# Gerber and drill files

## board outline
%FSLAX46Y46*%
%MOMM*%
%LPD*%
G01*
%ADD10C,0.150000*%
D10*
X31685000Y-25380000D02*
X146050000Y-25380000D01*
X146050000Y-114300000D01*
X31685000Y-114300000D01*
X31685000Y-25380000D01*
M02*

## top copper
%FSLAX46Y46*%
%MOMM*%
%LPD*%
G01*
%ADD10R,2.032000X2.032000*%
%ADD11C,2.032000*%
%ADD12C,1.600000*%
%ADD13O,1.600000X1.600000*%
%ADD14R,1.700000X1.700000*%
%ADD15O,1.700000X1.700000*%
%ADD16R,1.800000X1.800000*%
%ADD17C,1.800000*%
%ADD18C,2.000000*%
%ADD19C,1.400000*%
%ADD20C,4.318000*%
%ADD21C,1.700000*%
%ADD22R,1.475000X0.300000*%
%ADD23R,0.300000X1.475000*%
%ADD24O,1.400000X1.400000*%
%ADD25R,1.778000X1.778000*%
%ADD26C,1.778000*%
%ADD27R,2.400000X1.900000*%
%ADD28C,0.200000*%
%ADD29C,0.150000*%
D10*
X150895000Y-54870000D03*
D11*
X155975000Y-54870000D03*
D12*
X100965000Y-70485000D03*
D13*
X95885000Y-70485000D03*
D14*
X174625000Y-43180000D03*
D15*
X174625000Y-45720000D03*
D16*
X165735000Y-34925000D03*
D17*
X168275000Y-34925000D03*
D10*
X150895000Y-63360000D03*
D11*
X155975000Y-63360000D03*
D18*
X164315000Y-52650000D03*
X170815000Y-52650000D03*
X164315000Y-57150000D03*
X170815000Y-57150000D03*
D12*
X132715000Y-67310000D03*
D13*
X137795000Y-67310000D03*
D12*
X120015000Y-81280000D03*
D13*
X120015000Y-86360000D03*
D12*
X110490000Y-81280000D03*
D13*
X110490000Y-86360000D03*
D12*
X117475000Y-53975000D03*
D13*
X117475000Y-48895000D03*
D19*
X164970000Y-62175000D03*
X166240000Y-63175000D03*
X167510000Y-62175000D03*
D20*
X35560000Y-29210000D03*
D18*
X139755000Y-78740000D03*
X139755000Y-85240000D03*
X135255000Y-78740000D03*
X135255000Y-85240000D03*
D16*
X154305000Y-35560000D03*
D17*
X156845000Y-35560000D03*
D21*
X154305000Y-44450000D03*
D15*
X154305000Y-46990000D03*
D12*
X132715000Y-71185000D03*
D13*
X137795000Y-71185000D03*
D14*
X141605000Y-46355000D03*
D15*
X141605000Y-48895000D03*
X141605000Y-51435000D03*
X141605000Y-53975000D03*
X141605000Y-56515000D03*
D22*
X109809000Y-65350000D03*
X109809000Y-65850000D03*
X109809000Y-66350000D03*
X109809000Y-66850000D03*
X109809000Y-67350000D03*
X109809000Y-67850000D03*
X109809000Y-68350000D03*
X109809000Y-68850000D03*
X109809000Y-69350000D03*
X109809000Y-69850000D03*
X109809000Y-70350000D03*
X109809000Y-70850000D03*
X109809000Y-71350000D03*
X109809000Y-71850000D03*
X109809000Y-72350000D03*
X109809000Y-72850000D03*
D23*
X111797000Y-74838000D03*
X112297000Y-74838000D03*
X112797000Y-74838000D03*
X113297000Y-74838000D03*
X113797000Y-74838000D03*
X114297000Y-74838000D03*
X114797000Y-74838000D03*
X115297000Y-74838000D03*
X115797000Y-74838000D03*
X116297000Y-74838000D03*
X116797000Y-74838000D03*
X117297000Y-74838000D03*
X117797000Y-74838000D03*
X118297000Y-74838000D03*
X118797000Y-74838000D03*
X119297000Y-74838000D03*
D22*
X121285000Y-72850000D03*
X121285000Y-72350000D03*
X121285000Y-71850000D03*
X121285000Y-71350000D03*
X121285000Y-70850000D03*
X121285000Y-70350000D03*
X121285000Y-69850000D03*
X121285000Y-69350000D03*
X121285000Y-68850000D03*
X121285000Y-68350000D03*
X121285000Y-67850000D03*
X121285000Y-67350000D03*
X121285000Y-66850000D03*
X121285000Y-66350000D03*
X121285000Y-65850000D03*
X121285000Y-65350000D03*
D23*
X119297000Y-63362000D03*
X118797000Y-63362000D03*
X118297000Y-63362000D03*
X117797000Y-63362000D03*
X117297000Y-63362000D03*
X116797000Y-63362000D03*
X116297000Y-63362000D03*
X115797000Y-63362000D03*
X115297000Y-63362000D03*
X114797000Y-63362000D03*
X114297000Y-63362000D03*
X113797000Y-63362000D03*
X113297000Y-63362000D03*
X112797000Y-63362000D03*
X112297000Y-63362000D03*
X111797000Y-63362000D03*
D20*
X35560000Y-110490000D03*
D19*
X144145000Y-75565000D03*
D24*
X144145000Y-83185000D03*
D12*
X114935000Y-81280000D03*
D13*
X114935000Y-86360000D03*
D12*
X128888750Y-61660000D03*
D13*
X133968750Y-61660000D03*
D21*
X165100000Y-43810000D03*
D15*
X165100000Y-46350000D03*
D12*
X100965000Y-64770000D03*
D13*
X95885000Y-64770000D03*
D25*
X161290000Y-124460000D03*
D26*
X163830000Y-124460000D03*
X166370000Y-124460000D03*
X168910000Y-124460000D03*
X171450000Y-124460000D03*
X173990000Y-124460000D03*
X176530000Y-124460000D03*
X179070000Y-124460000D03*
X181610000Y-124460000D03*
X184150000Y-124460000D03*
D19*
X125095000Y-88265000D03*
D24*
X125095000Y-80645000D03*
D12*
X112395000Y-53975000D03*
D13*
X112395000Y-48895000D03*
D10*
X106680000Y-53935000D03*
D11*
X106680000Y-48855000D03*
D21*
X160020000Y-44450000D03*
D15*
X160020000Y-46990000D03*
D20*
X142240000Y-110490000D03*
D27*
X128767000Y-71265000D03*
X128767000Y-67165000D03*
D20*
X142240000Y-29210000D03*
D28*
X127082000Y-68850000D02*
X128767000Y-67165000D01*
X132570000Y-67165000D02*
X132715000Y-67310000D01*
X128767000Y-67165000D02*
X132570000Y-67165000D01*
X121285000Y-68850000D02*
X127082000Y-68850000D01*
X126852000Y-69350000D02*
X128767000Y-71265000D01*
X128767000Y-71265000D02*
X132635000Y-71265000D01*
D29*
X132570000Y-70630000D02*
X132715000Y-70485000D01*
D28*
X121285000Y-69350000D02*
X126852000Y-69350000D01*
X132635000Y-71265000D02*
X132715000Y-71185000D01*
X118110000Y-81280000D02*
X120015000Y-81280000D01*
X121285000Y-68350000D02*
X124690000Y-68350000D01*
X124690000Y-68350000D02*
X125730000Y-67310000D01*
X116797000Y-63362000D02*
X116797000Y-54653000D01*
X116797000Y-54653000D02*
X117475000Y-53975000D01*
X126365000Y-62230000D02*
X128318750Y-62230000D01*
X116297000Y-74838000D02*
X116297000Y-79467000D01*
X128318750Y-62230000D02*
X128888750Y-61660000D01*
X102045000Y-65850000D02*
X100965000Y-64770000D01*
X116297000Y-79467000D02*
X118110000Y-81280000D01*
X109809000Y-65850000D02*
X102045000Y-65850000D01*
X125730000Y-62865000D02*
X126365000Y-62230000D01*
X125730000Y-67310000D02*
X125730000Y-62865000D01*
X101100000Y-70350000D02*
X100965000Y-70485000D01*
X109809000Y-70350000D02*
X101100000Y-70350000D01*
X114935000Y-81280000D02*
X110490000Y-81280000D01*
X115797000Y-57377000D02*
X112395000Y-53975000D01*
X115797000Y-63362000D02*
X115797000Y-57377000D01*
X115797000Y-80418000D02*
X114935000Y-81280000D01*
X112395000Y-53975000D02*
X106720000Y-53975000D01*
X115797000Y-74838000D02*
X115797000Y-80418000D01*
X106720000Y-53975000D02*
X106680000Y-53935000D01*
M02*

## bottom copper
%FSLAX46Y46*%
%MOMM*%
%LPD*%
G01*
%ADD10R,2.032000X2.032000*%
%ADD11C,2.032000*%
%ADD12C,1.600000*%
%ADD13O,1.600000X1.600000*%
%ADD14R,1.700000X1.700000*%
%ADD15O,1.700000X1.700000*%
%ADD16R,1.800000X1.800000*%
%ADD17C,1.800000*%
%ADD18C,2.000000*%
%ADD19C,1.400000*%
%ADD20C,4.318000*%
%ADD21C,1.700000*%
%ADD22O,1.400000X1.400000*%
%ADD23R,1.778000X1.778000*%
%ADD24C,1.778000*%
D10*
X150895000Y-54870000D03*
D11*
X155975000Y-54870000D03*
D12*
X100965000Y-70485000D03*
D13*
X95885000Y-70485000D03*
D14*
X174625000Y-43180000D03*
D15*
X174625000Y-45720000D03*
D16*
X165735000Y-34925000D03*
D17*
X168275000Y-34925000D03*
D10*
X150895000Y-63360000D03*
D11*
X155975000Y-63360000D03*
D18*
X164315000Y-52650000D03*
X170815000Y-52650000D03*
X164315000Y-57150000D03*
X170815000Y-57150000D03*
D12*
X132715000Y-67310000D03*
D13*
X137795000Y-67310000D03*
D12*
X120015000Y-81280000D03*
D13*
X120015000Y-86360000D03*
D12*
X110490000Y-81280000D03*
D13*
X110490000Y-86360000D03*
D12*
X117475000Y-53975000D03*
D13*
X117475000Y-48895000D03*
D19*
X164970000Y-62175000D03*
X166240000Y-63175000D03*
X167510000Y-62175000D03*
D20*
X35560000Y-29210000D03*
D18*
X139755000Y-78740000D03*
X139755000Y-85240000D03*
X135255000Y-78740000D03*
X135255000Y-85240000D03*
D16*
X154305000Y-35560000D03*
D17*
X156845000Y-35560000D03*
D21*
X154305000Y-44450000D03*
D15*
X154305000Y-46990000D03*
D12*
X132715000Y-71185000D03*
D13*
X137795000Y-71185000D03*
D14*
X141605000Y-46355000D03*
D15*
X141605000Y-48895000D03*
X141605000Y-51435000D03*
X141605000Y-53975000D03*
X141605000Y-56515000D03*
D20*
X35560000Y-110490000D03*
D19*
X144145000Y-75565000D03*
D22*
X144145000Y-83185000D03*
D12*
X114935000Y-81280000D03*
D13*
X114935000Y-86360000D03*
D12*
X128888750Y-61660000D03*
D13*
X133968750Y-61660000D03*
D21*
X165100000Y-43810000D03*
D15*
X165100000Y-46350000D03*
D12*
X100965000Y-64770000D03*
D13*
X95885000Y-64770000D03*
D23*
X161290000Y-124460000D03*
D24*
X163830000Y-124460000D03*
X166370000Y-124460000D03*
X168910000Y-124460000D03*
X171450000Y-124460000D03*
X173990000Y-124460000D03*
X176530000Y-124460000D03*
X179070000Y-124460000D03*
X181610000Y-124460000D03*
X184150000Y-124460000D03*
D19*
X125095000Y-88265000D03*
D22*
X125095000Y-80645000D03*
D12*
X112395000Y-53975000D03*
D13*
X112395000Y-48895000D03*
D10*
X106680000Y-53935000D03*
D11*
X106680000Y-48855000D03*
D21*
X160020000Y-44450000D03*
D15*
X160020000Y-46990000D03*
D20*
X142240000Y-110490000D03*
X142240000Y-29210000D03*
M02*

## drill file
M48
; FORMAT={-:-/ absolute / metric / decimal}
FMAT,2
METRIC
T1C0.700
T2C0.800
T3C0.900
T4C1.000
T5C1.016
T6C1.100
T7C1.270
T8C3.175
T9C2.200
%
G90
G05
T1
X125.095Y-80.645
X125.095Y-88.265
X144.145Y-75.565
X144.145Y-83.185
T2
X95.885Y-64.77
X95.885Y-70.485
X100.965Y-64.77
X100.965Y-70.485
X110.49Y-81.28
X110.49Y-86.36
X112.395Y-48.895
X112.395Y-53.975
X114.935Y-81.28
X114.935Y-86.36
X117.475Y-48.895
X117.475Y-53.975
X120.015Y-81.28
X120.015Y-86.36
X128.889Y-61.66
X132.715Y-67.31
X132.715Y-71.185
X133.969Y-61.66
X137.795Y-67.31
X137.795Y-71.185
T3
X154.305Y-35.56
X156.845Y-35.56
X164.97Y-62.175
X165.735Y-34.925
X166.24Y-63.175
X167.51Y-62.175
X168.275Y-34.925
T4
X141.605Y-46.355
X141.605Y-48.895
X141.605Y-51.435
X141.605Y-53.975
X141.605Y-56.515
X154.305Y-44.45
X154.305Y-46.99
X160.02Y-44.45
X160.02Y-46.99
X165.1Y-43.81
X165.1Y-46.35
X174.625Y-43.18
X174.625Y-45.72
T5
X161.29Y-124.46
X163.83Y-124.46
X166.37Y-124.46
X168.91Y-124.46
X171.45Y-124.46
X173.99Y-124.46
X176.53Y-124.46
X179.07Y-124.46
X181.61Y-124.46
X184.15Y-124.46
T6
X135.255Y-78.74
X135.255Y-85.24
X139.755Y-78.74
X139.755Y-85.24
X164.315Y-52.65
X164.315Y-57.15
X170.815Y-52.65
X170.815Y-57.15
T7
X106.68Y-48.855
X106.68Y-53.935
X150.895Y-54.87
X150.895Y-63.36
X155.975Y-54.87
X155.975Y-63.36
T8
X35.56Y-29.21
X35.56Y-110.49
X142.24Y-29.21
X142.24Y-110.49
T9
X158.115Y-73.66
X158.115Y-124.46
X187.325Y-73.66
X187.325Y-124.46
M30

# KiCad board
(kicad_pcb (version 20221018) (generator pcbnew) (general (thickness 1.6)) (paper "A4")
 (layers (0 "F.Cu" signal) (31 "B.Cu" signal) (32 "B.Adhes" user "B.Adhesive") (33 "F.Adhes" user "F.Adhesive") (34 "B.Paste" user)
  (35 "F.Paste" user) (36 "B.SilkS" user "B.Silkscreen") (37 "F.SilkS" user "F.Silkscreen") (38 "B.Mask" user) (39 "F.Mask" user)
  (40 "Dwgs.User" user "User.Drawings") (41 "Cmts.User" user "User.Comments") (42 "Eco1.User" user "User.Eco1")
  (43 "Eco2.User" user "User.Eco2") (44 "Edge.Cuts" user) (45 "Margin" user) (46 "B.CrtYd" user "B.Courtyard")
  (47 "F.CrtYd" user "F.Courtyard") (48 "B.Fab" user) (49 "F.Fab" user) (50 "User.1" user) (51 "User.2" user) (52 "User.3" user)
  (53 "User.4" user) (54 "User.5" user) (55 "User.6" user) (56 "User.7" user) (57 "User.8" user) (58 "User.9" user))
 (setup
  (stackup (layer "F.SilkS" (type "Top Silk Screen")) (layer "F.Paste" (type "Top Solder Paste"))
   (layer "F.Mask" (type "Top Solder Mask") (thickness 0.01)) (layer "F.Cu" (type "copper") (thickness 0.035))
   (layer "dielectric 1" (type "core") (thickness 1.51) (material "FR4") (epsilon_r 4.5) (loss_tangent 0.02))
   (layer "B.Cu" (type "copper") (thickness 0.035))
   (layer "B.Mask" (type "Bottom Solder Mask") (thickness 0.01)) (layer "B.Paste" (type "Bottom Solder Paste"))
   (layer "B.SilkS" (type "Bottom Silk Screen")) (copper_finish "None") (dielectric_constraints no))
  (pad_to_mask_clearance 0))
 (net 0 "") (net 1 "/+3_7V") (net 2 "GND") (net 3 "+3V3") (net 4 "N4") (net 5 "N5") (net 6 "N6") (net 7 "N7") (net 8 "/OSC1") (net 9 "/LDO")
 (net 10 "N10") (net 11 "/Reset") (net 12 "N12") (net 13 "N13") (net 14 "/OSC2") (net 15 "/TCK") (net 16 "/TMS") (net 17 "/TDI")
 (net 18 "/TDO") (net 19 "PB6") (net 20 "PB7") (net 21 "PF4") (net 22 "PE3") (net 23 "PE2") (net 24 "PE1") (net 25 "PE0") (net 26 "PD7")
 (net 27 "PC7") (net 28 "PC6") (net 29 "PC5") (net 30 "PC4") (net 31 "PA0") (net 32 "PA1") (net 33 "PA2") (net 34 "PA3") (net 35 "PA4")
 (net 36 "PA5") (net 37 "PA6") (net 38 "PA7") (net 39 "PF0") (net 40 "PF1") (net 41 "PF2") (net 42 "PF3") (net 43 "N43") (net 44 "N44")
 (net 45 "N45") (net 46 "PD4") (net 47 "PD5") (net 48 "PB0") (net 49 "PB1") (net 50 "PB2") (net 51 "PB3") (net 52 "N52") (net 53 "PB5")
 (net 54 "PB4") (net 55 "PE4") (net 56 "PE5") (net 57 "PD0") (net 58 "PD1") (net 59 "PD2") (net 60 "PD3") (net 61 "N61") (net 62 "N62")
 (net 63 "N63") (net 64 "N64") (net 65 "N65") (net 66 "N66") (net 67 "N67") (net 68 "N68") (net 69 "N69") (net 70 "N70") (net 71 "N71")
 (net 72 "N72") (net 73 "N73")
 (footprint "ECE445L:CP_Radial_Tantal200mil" (layer "F.Cu") (at 150.895 54.87)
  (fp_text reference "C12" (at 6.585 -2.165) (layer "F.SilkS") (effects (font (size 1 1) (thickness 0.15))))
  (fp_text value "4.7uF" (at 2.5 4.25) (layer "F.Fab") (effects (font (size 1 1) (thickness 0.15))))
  (pad "1" thru_hole rect (at 0 0) (size 2.032 2.032) (drill 1.27) (layers "*.Cu" "*.Mask") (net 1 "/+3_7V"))
  (pad "2" thru_hole circle (at 5.08 0) (size 2.032 2.032) (drill 1.27) (layers "*.Cu" "*.Mask") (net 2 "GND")))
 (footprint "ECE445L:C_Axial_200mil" (layer "F.Cu") (at 100.965 70.485 180)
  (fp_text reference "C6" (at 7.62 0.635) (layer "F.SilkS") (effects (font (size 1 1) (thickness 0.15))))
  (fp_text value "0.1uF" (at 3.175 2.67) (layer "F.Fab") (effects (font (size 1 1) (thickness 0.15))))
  (pad "1" thru_hole circle (at 0 0 180) (size 1.6 1.6) (drill 0.8) (layers "*.Cu" "*.Mask") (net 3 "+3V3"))
  (pad "2" thru_hole oval (at 5.08 0 180) (size 1.6 1.6) (drill 0.8) (layers "*.Cu" "*.Mask") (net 2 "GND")))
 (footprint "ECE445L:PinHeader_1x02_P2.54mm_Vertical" (layer "F.Cu") (at 174.625 43.18)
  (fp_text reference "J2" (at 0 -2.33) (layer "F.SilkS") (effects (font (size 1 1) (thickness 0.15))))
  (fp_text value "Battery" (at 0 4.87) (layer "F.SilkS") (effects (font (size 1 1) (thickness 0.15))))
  (pad "1" thru_hole rect (at 0 0) (size 1.7 1.7) (drill 1) (layers "*.Cu" "*.Mask") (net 2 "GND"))
  (pad "2" thru_hole oval (at 0 2.54) (size 1.7 1.7) (drill 1) (layers "*.Cu" "*.Mask") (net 1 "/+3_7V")))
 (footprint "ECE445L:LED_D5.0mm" (layer "F.Cu") (at 165.735 34.925)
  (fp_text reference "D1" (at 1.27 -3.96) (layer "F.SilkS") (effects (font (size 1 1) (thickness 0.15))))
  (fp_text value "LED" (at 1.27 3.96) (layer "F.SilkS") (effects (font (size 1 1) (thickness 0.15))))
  (pad "1" thru_hole rect (at 0 0) (size 1.8 1.8) (drill 0.9) (layers "*.Cu" "*.Mask") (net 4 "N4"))
  (pad "2" thru_hole circle (at 2.54 0) (size 1.8 1.8) (drill 0.9) (layers "*.Cu" "*.Mask") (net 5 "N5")))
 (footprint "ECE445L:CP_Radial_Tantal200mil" (layer "F.Cu") (at 150.895 63.36)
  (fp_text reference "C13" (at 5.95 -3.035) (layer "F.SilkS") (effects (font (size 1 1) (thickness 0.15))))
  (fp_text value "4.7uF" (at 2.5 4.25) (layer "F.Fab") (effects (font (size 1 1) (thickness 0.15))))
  (pad "1" thru_hole rect (at 0 0) (size 2.032 2.032) (drill 1.27) (layers "*.Cu" "*.Mask") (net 3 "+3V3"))
  (pad "2" thru_hole circle (at 5.08 0) (size 2.032 2.032) (drill 1.27) (layers "*.Cu" "*.Mask") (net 2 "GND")))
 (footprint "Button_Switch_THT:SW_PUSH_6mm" (layer "F.Cu") (at 164.315 52.65)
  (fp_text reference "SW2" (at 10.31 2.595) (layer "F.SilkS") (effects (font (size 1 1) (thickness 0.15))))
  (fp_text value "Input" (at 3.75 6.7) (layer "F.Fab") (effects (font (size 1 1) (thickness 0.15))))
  (pad "1" thru_hole circle (at 0 0 90) (size 2 2) (drill 1.1) (layers "*.Cu" "*.Mask") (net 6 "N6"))
  (pad "1" thru_hole circle (at 6.5 0 90) (size 2 2) (drill 1.1) (layers "*.Cu" "*.Mask") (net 6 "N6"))
  (pad "2" thru_hole circle (at 0 4.5 90) (size 2 2) (drill 1.1) (layers "*.Cu" "*.Mask") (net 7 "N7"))
  (pad "2" thru_hole circle (at 6.5 4.5 90) (size 2 2) (drill 1.1) (layers "*.Cu" "*.Mask") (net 7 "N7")))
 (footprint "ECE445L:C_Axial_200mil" (layer "F.Cu") (at 132.715 67.31)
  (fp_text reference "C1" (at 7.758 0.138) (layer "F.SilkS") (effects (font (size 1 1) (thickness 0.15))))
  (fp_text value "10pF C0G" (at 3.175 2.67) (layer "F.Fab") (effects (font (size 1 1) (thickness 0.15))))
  (pad "1" thru_hole circle (at 0 0) (size 1.6 1.6) (drill 0.8) (layers "*.Cu" "*.Mask") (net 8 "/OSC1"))
  (pad "2" thru_hole oval (at 5.08 0) (size 1.6 1.6) (drill 0.8) (layers "*.Cu" "*.Mask") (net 2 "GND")))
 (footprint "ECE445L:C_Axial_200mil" (layer "F.Cu") (at 120.015 81.28 -90)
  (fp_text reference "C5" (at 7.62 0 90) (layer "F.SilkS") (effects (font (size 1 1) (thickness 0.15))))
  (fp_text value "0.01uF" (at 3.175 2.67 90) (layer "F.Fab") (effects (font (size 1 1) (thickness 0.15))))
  (pad "1" thru_hole circle (at 0 0 270) (size 1.6 1.6) (drill 0.8) (layers "*.Cu" "*.Mask") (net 3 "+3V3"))
  (pad "2" thru_hole oval (at 5.08 0 270) (size 1.6 1.6) (drill 0.8) (layers "*.Cu" "*.Mask") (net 2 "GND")))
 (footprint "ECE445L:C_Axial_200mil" (layer "F.Cu") (at 110.49 81.28 -90)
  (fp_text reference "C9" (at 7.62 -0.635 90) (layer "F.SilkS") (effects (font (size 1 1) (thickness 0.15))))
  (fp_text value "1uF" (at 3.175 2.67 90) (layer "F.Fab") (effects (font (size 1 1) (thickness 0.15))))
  (pad "1" thru_hole circle (at 0 0 270) (size 1.6 1.6) (drill 0.8) (layers "*.Cu" "*.Mask") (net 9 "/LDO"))
  (pad "2" thru_hole oval (at 5.08 0 270) (size 1.6 1.6) (drill 0.8) (layers "*.Cu" "*.Mask") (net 2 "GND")))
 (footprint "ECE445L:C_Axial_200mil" (layer "F.Cu") (at 117.475 53.975 90)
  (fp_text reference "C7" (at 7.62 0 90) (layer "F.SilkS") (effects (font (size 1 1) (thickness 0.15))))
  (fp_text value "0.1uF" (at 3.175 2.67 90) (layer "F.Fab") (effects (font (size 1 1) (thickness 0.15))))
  (pad "1" thru_hole circle (at 0 0 90) (size 1.6 1.6) (drill 0.8) (layers "*.Cu" "*.Mask") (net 3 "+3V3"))
  (pad "2" thru_hole oval (at 5.08 0 90) (size 1.6 1.6) (drill 0.8) (layers "*.Cu" "*.Mask") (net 2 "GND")))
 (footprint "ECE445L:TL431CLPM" (layer "F.Cu") (at 164.97 62.175)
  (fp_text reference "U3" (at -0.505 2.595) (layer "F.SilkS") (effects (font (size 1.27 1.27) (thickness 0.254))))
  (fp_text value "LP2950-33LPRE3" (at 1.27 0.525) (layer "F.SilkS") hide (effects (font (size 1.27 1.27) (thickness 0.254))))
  (pad "1" thru_hole circle (at 0 0) (size 1.4 1.4) (drill 0.9) (layers "*.Cu" "*.Mask") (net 3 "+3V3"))
  (pad "2" thru_hole circle (at 1.27 1) (size 1.4 1.4) (drill 0.9) (layers "*.Cu" "*.Mask") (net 2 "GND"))
  (pad "3" thru_hole circle (at 2.54 0) (size 1.4 1.4) (drill 0.9) (layers "*.Cu" "*.Mask") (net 1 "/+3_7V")))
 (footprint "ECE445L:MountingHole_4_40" (layer "F.Cu") (at 35.56 29.21)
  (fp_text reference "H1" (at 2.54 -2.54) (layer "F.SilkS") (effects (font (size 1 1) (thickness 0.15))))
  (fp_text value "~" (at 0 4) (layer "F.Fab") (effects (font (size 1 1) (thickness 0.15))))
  (pad "1" thru_hole circle (at 0 0) (size 4.318 4.318) (drill 3.175) (layers "*.Cu" "*.Mask") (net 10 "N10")))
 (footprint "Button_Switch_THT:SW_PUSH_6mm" (layer "F.Cu") (at 139.755 78.74 -90)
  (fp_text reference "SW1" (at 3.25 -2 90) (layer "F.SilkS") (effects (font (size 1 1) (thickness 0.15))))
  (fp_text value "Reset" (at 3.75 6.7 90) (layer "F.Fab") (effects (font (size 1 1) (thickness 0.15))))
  (pad "1" thru_hole circle (at 0 0) (size 2 2) (drill 1.1) (layers "*.Cu" "*.Mask") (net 2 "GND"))
  (pad "1" thru_hole circle (at 6.5 0) (size 2 2) (drill 1.1) (layers "*.Cu" "*.Mask") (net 2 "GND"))
  (pad "2" thru_hole circle (at 0 4.5) (size 2 2) (drill 1.1) (layers "*.Cu" "*.Mask") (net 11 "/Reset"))
  (pad "2" thru_hole circle (at 6.5 4.5) (size 2 2) (drill 1.1) (layers "*.Cu" "*.Mask") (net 11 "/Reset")))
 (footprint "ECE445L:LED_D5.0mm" (layer "F.Cu") (at 154.305 35.56)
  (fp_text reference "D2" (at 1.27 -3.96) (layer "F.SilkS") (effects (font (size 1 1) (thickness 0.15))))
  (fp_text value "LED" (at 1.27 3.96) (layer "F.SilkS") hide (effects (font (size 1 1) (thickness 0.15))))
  (pad "1" thru_hole rect (at 0 0) (size 1.8 1.8) (drill 0.9) (layers "*.Cu" "*.Mask") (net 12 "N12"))
  (pad "2" thru_hole circle (at 2.54 0) (size 1.8 1.8) (drill 0.9) (layers "*.Cu" "*.Mask") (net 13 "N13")))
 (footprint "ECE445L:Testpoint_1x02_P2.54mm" (layer "F.Cu") (at 154.305 44.45)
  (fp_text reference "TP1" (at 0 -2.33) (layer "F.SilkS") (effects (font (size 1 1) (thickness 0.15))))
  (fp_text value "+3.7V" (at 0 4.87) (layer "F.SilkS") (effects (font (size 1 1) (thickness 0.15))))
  (pad "1" thru_hole circle (at 0 0) (size 1.7 1.7) (drill 1) (layers "*.Cu" "*.Mask") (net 1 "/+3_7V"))
  (pad "2" thru_hole oval (at 0 2.54) (size 1.7 1.7) (drill 1) (layers "*.Cu" "*.Mask") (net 1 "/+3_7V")))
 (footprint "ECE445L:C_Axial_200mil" (layer "F.Cu") (at 132.715 71.185)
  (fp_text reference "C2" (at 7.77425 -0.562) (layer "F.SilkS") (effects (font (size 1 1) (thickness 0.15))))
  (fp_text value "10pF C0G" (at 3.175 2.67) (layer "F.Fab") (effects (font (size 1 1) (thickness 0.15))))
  (pad "1" thru_hole circle (at 0 0) (size 1.6 1.6) (drill 0.8) (layers "*.Cu" "*.Mask") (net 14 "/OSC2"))
  (pad "2" thru_hole oval (at 5.08 0) (size 1.6 1.6) (drill 0.8) (layers "*.Cu" "*.Mask") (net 2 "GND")))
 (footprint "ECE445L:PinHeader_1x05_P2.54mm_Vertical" (layer "F.Cu") (at 141.605 46.355)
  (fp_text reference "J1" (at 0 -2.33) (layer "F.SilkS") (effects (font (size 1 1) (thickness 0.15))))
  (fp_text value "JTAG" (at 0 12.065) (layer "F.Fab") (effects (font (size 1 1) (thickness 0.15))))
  (pad "1" thru_hole rect (at 0 0) (size 1.7 1.7) (drill 1) (layers "*.Cu" "*.Mask") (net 2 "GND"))
  (pad "2" thru_hole oval (at 0 2.54) (size 1.7 1.7) (drill 1) (layers "*.Cu" "*.Mask") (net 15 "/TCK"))
  (pad "3" thru_hole oval (at 0 5.08) (size 1.7 1.7) (drill 1) (layers "*.Cu" "*.Mask") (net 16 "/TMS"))
  (pad "4" thru_hole oval (at 0 7.62) (size 1.7 1.7) (drill 1) (layers "*.Cu" "*.Mask") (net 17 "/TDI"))
  (pad "5" thru_hole oval (at 0 10.16) (size 1.7 1.7) (drill 1) (layers "*.Cu" "*.Mask") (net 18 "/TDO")))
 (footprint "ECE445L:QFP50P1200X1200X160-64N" (layer "F.Cu") (at 115.547 69.1)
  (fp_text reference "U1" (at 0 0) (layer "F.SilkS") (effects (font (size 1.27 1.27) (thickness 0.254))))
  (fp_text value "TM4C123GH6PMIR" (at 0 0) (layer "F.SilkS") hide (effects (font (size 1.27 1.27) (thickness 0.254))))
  (pad "1" smd rect (at -5.738 -3.75 90) (size 0.3 1.475) (layers "F.Cu" "F.Paste" "F.Mask") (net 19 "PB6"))
  (pad "2" smd rect (at -5.738 -3.25 90) (size 0.3 1.475) (layers "F.Cu" "F.Paste" "F.Mask") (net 3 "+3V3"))
  (pad "3" smd rect (at -5.738 -2.75 90) (size 0.3 1.475) (layers "F.Cu" "F.Paste" "F.Mask") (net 2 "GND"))
  (pad "4" smd rect (at -5.738 -2.25 90) (size 0.3 1.475) (layers "F.Cu" "F.Paste" "F.Mask") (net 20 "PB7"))
  (pad "5" smd rect (at -5.738 -1.75 90) (size 0.3 1.475) (layers "F.Cu" "F.Paste" "F.Mask") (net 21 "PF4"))
  (pad "6" smd rect (at -5.738 -1.25 90) (size 0.3 1.475) (layers "F.Cu" "F.Paste" "F.Mask") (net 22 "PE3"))
  (pad "7" smd rect (at -5.738 -0.75 90) (size 0.3 1.475) (layers "F.Cu" "F.Paste" "F.Mask") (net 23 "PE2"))
  (pad "8" smd rect (at -5.738 -0.25 90) (size 0.3 1.475) (layers "F.Cu" "F.Paste" "F.Mask") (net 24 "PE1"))
  (pad "9" smd rect (at -5.738 0.25 90) (size 0.3 1.475) (layers "F.Cu" "F.Paste" "F.Mask") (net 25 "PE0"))
  (pad "10" smd rect (at -5.738 0.75 90) (size 0.3 1.475) (layers "F.Cu" "F.Paste" "F.Mask") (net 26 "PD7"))
  (pad "11" smd rect (at -5.738 1.25 90) (size 0.3 1.475) (layers "F.Cu" "F.Paste" "F.Mask") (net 3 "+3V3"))
  (pad "12" smd rect (at -5.738 1.75 90) (size 0.3 1.475) (layers "F.Cu" "F.Paste" "F.Mask") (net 2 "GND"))
  (pad "13" smd rect (at -5.738 2.25 90) (size 0.3 1.475) (layers "F.Cu" "F.Paste" "F.Mask") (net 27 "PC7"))
  (pad "14" smd rect (at -5.738 2.75 90) (size 0.3 1.475) (layers "F.Cu" "F.Paste" "F.Mask") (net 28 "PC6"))
  (pad "15" smd rect (at -5.738 3.25 90) (size 0.3 1.475) (layers "F.Cu" "F.Paste" "F.Mask") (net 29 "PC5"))
  (pad "16" smd rect (at -5.738 3.75 90) (size 0.3 1.475) (layers "F.Cu" "F.Paste" "F.Mask") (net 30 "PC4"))
  (pad "17" smd rect (at -3.75 5.738) (size 0.3 1.475) (layers "F.Cu" "F.Paste" "F.Mask") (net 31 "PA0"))
  (pad "18" smd rect (at -3.25 5.738) (size 0.3 1.475) (layers "F.Cu" "F.Paste" "F.Mask") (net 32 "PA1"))
  (pad "19" smd rect (at -2.75 5.738) (size 0.3 1.475) (layers "F.Cu" "F.Paste" "F.Mask") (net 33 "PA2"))
  (pad "20" smd rect (at -2.25 5.738) (size 0.3 1.475) (layers "F.Cu" "F.Paste" "F.Mask") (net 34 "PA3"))
  (pad "21" smd rect (at -1.75 5.738) (size 0.3 1.475) (layers "F.Cu" "F.Paste" "F.Mask") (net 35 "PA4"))
  (pad "22" smd rect (at -1.25 5.738) (size 0.3 1.475) (layers "F.Cu" "F.Paste" "F.Mask") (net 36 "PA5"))
  (pad "23" smd rect (at -0.75 5.738) (size 0.3 1.475) (layers "F.Cu" "F.Paste" "F.Mask") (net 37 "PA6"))
  (pad "24" smd rect (at -0.25 5.738) (size 0.3 1.475) (layers "F.Cu" "F.Paste" "F.Mask") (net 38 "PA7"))
  (pad "25" smd rect (at 0.25 5.738) (size 0.3 1.475) (layers "F.Cu" "F.Paste" "F.Mask") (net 9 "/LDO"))
  (pad "26" smd rect (at 0.75 5.738) (size 0.3 1.475) (layers "F.Cu" "F.Paste" "F.Mask") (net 3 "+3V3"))
  (pad "27" smd rect (at 1.25 5.738) (size 0.3 1.475) (layers "F.Cu" "F.Paste" "F.Mask") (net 2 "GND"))
  (pad "28" smd rect (at 1.75 5.738) (size 0.3 1.475) (layers "F.Cu" "F.Paste" "F.Mask") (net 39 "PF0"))
  (pad "29" smd rect (at 2.25 5.738) (size 0.3 1.475) (layers "F.Cu" "F.Paste" "F.Mask") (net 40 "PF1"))
  (pad "30" smd rect (at 2.75 5.738) (size 0.3 1.475) (layers "F.Cu" "F.Paste" "F.Mask") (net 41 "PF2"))
  (pad "31" smd rect (at 3.25 5.738) (size 0.3 1.475) (layers "F.Cu" "F.Paste" "F.Mask") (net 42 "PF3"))
  (pad "32" smd rect (at 3.75 5.738) (size 0.3 1.475) (layers "F.Cu" "F.Paste" "F.Mask") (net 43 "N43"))
  (pad "33" smd rect (at 5.738 3.75 90) (size 0.3 1.475) (layers "F.Cu" "F.Paste" "F.Mask") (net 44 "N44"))
  (pad "34" smd rect (at 5.738 3.25 90) (size 0.3 1.475) (layers "F.Cu" "F.Paste" "F.Mask") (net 2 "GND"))
  (pad "35" smd rect (at 5.738 2.75 90) (size 0.3 1.475) (layers "F.Cu" "F.Paste" "F.Mask") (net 2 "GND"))
  (pad "36" smd rect (at 5.738 2.25 90) (size 0.3 1.475) (layers "F.Cu" "F.Paste" "F.Mask") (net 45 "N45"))
  (pad "37" smd rect (at 5.738 1.75 90) (size 0.3 1.475) (layers "F.Cu" "F.Paste" "F.Mask") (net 3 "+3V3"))
  (pad "38" smd rect (at 5.738 1.25 90) (size 0.3 1.475) (layers "F.Cu" "F.Paste" "F.Mask") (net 11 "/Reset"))
  (pad "39" smd rect (at 5.738 0.75 90) (size 0.3 1.475) (layers "F.Cu" "F.Paste" "F.Mask") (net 2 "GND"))
  (pad "40" smd rect (at 5.738 0.25 90) (size 0.3 1.475) (layers "F.Cu" "F.Paste" "F.Mask") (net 14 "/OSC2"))
  (pad "41" smd rect (at 5.738 -0.25 90) (size 0.3 1.475) (layers "F.Cu" "F.Paste" "F.Mask") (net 8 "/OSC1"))
  (pad "42" smd rect (at 5.738 -0.75 90) (size 0.3 1.475) (layers "F.Cu" "F.Paste" "F.Mask") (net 3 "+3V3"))
  (pad "43" smd rect (at 5.738 -1.25 90) (size 0.3 1.475) (layers "F.Cu" "F.Paste" "F.Mask") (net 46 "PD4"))
  (pad "44" smd rect (at 5.738 -1.75 90) (size 0.3 1.475) (layers "F.Cu" "F.Paste" "F.Mask") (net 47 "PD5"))
  (pad "45" smd rect (at 5.738 -2.25 90) (size 0.3 1.475) (layers "F.Cu" "F.Paste" "F.Mask") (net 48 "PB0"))
  (pad "46" smd rect (at 5.738 -2.75 90) (size 0.3 1.475) (layers "F.Cu" "F.Paste" "F.Mask") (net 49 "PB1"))
  (pad "47" smd rect (at 5.738 -3.25 90) (size 0.3 1.475) (layers "F.Cu" "F.Paste" "F.Mask") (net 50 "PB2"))
  (pad "48" smd rect (at 5.738 -3.75 90) (size 0.3 1.475) (layers "F.Cu" "F.Paste" "F.Mask") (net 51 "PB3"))
  (pad "49" smd rect (at 3.75 -5.738) (size 0.3 1.475) (layers "F.Cu" "F.Paste" "F.Mask") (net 18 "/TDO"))
  (pad "50" smd rect (at 3.25 -5.738) (size 0.3 1.475) (layers "F.Cu" "F.Paste" "F.Mask") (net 17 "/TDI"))
  (pad "51" smd rect (at 2.75 -5.738) (size 0.3 1.475) (layers "F.Cu" "F.Paste" "F.Mask") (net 16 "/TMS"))
  (pad "52" smd rect (at 2.25 -5.738) (size 0.3 1.475) (layers "F.Cu" "F.Paste" "F.Mask") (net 15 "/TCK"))
  (pad "53" smd rect (at 1.75 -5.738) (size 0.3 1.475) (layers "F.Cu" "F.Paste" "F.Mask") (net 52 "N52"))
  (pad "54" smd rect (at 1.25 -5.738) (size 0.3 1.475) (layers "F.Cu" "F.Paste" "F.Mask") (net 3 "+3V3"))
  (pad "55" smd rect (at 0.75 -5.738) (size 0.3 1.475) (layers "F.Cu" "F.Paste" "F.Mask") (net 2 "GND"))
  (pad "56" smd rect (at 0.25 -5.738) (size 0.3 1.475) (layers "F.Cu" "F.Paste" "F.Mask") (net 9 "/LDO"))
  (pad "57" smd rect (at -0.25 -5.738) (size 0.3 1.475) (layers "F.Cu" "F.Paste" "F.Mask") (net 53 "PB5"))
  (pad "58" smd rect (at -0.75 -5.738) (size 0.3 1.475) (layers "F.Cu" "F.Paste" "F.Mask") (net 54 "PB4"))
  (pad "59" smd rect (at -1.25 -5.738) (size 0.3 1.475) (layers "F.Cu" "F.Paste" "F.Mask") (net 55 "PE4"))
  (pad "60" smd rect (at -1.75 -5.738) (size 0.3 1.475) (layers "F.Cu" "F.Paste" "F.Mask") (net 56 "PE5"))
  (pad "61" smd rect (at -2.25 -5.738) (size 0.3 1.475) (layers "F.Cu" "F.Paste" "F.Mask") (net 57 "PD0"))
  (pad "62" smd rect (at -2.75 -5.738) (size 0.3 1.475) (layers "F.Cu" "F.Paste" "F.Mask") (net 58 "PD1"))
  (pad "63" smd rect (at -3.25 -5.738) (size 0.3 1.475) (layers "F.Cu" "F.Paste" "F.Mask") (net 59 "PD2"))
  (pad "64" smd rect (at -3.75 -5.738) (size 0.3 1.475) (layers "F.Cu" "F.Paste" "F.Mask") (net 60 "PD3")))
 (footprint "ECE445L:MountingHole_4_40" (layer "F.Cu") (at 35.56 110.49)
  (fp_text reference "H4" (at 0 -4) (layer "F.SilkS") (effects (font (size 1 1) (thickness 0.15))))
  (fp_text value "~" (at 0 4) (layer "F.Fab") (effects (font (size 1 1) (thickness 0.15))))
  (pad "1" thru_hole circle (at 0 0) (size 4.318 4.318) (drill 3.175) (layers "*.Cu" "*.Mask") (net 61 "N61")))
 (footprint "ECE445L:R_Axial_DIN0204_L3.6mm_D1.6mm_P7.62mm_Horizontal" (layer "F.Cu") (at 144.145 75.565 -90)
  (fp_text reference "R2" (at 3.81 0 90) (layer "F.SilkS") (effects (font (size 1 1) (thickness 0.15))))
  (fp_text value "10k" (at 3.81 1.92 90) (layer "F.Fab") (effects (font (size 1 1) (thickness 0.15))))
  (pad "1" thru_hole circle (at 0 0 270) (size 1.4 1.4) (drill 0.7) (layers "*.Cu" "*.Mask") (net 3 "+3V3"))
  (pad "2" thru_hole oval (at 7.62 0 270) (size 1.4 1.4) (drill 0.7) (layers "*.Cu" "*.Mask") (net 11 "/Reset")))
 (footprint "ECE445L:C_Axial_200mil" (layer "F.Cu") (at 114.935 81.28 -90)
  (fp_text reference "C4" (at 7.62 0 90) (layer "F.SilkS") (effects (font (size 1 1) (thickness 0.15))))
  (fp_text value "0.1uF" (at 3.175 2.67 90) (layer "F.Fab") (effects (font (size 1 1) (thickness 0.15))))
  (pad "1" thru_hole circle (at 0 0 270) (size 1.6 1.6) (drill 0.8) (layers "*.Cu" "*.Mask") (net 9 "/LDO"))
  (pad "2" thru_hole oval (at 5.08 0 270) (size 1.6 1.6) (drill 0.8) (layers "*.Cu" "*.Mask") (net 2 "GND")))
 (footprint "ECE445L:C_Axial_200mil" (layer "F.Cu") (at 128.88875 61.66)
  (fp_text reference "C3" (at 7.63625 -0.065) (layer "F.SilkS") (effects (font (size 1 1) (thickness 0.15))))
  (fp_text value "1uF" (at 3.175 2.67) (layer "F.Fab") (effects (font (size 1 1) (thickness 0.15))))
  (pad "1" thru_hole circle (at 0 0) (size 1.6 1.6) (drill 0.8) (layers "*.Cu" "*.Mask") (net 3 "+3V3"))
  (pad "2" thru_hole oval (at 5.08 0) (size 1.6 1.6) (drill 0.8) (layers "*.Cu" "*.Mask") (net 2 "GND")))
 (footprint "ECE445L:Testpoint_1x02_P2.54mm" (layer "F.Cu") (at 165.1 43.81)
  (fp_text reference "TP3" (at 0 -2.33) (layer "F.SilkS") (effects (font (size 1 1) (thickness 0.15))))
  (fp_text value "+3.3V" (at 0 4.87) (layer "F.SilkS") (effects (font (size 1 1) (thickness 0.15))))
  (pad "1" thru_hole circle (at 0 0) (size 1.7 1.7) (drill 1) (layers "*.Cu" "*.Mask") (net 3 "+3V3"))
  (pad "2" thru_hole oval (at 0 2.54) (size 1.7 1.7) (drill 1) (layers "*.Cu" "*.Mask") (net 3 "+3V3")))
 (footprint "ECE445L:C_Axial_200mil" (layer "F.Cu") (at 100.965 64.77 180)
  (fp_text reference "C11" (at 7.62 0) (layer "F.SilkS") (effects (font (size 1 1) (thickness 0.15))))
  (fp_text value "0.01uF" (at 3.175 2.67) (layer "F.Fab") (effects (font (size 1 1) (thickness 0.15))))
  (pad "1" thru_hole circle (at 0 0 180) (size 1.6 1.6) (drill 0.8) (layers "*.Cu" "*.Mask") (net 3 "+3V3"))
  (pad "2" thru_hole oval (at 5.08 0 180) (size 1.6 1.6) (drill 0.8) (layers "*.Cu" "*.Mask") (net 2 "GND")))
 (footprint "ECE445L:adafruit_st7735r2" (layer "F.Cu") (at 172.72 99.06)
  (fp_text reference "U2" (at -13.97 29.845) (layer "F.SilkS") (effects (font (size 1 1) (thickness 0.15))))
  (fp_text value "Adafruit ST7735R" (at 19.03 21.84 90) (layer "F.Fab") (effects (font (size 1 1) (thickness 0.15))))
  (pad "" np_thru_hole circle (at -14.605 -25.4 90) (size 2.2 2.2) (drill 2.2) (layers "*.Cu" "*.Mask"))
  (pad "" np_thru_hole circle (at -14.605 25.4 90) (size 2.2 2.2) (drill 2.2) (layers "F&B.Cu" "*.Mask"))
  (pad "" np_thru_hole circle (at 14.605 -25.4 90) (size 2.2 2.2) (drill 2.2) (layers "F&B.Cu" "*.Mask"))
  (pad "" np_thru_hole circle (at 14.605 25.4 90) (size 2.2 2.2) (drill 2.2) (layers "F&B.Cu" "*.Mask"))
  (pad "1" thru_hole rect (at -11.43 25.4 90) (size 1.778 1.778) (drill 1.016) (layers "*.Cu" "*.Mask") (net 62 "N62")
   (solder_mask_margin 0.102))
  (pad "2" thru_hole circle (at -8.89 25.4 90) (size 1.778 1.778) (drill 1.016) (layers "*.Cu" "*.Mask") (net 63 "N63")
   (solder_mask_margin 0.102))
  (pad "3" thru_hole circle (at -6.35 25.4 90) (size 1.778 1.778) (drill 1.016) (layers "*.Cu" "*.Mask") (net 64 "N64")
   (solder_mask_margin 0.102))
  (pad "4" thru_hole circle (at -3.81 25.4 90) (size 1.778 1.778) (drill 1.016) (layers "*.Cu" "*.Mask") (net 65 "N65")
   (solder_mask_margin 0.102))
  (pad "5" thru_hole circle (at -1.27 25.4 90) (size 1.778 1.778) (drill 1.016) (layers "*.Cu" "*.Mask") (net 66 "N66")
   (solder_mask_margin 0.102))
  (pad "6" thru_hole circle (at 1.27 25.4 90) (size 1.778 1.778) (drill 1.016) (layers "*.Cu" "*.Mask") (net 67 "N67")
   (solder_mask_margin 0.102))
  (pad "7" thru_hole circle (at 3.81 25.4 90) (size 1.778 1.778) (drill 1.016) (layers "*.Cu" "*.Mask") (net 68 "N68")
   (solder_mask_margin 0.102))
  (pad "8" thru_hole circle (at 6.35 25.4 90) (size 1.778 1.778) (drill 1.016) (layers "*.Cu" "*.Mask") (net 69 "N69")
   (solder_mask_margin 0.102))
  (pad "9" thru_hole circle (at 8.89 25.4 90) (size 1.778 1.778) (drill 1.016) (layers "*.Cu" "*.Mask") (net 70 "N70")
   (solder_mask_margin 0.102))
  (pad "10" thru_hole circle (at 11.43 25.4 90) (size 1.778 1.778) (drill 1.016) (layers "*.Cu" "*.Mask") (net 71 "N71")
   (solder_mask_margin 0.102)))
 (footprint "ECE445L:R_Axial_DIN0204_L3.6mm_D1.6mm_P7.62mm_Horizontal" (layer "F.Cu") (at 125.095 88.265 90)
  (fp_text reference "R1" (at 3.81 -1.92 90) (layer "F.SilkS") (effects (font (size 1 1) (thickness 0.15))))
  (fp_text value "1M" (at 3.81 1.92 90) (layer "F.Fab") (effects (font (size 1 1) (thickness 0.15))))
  (pad "1" thru_hole circle (at 0 0 90) (size 1.4 1.4) (drill 0.7) (layers "*.Cu" "*.Mask") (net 3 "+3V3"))
  (pad "2" thru_hole oval (at 7.62 0 90) (size 1.4 1.4) (drill 0.7) (layers "*.Cu" "*.Mask") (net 43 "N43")))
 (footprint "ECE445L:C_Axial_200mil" (layer "F.Cu") (at 112.395 53.975 90)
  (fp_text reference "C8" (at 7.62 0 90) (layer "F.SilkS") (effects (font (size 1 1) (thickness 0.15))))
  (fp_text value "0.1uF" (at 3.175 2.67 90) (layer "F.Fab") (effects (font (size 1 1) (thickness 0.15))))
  (pad "1" thru_hole circle (at 0 0 90) (size 1.6 1.6) (drill 0.8) (layers "*.Cu" "*.Mask") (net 9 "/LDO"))
  (pad "2" thru_hole oval (at 5.08 0 90) (size 1.6 1.6) (drill 0.8) (layers "*.Cu" "*.Mask") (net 2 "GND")))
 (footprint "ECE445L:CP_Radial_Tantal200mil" (layer "F.Cu") (at 106.68 53.935 90)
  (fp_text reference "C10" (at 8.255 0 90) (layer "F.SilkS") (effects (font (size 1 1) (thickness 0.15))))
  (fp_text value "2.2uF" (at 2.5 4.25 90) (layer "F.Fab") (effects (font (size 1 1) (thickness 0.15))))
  (pad "1" thru_hole rect (at 0 0 90) (size 2.032 2.032) (drill 1.27) (layers "*.Cu" "*.Mask") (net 9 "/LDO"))
  (pad "2" thru_hole circle (at 5.08 0 90) (size 2.032 2.032) (drill 1.27) (layers "*.Cu" "*.Mask") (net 2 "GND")))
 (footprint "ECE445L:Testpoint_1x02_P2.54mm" (layer "F.Cu") (at 160.02 44.45)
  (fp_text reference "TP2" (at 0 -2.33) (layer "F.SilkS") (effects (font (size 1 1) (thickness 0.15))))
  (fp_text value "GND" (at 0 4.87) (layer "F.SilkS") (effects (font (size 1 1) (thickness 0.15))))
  (pad "1" thru_hole circle (at 0 0) (size 1.7 1.7) (drill 1) (layers "*.Cu" "*.Mask") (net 2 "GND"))
  (pad "2" thru_hole oval (at 0 2.54) (size 1.7 1.7) (drill 1) (layers "*.Cu" "*.Mask") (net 2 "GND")))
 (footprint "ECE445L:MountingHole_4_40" (layer "F.Cu") (at 142.24 110.49)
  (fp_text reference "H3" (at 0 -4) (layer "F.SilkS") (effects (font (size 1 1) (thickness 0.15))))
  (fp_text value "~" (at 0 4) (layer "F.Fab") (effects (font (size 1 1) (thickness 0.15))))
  (pad "1" thru_hole circle (at 0 0) (size 4.318 4.318) (drill 3.175) (layers "*.Cu" "*.Mask") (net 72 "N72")))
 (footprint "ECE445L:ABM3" (layer "F.Cu") (at 128.767 69.215 90)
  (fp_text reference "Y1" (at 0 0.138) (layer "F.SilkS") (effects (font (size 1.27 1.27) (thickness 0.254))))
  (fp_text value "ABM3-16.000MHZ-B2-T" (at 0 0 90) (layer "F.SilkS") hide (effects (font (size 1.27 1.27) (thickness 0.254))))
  (pad "1" smd rect (at -2.05 0 90) (size 1.9 2.4) (layers "F.Cu" "F.Paste" "F.Mask") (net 14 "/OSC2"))
  (pad "2" smd rect (at 2.05 0 90) (size 1.9 2.4) (layers "F.Cu" "F.Paste" "F.Mask") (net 8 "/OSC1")))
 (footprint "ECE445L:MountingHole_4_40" (layer "F.Cu") (at 142.24 29.21)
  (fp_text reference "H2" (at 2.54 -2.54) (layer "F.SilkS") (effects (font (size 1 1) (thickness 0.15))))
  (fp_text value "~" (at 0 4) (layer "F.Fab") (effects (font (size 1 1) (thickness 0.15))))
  (pad "1" thru_hole circle (at 0 0) (size 4.318 4.318) (drill 3.175) (layers "*.Cu" "*.Mask") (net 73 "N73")))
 (gr_rect (start 31.685 25.38) (end 146.05 114.3) (stroke (width 0.15) (type default)) (fill none) (layer "Edge.Cuts"))
 (segment (start 127.082 68.85) (end 128.767 67.165) (width 0.2) (layer "F.Cu") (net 8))
 (segment (start 132.57 67.165) (end 132.715 67.31) (width 0.2) (layer "F.Cu") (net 8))
 (segment (start 128.767 67.165) (end 132.57 67.165) (width 0.2) (layer "F.Cu") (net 8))
 (segment (start 121.285 68.85) (end 127.082 68.85) (width 0.2) (layer "F.Cu") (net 8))
 (segment (start 126.852 69.35) (end 128.767 71.265) (width 0.2) (layer "F.Cu") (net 14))
 (segment (start 128.767 71.265) (end 132.635 71.265) (width 0.2) (layer "F.Cu") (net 14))
 (segment (start 132.57 70.63) (end 132.715 70.485) (width 0.15) (layer "F.Cu") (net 14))
 (segment (start 121.285 69.35) (end 126.852 69.35) (width 0.2) (layer "F.Cu") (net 14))
 (segment (start 132.635 71.265) (end 132.715 71.185) (width 0.2) (layer "F.Cu") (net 14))
 (segment (start 118.11 81.28) (end 120.015 81.28) (width 0.2) (layer "F.Cu") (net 3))
 (segment (start 121.285 68.35) (end 124.69 68.35) (width 0.2) (layer "F.Cu") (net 3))
 (segment (start 124.69 68.35) (end 125.73 67.31) (width 0.2) (layer "F.Cu") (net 3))
 (segment (start 116.797 63.362) (end 116.797 54.653) (width 0.2) (layer "F.Cu") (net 3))
 (segment (start 116.797 54.653) (end 117.475 53.975) (width 0.2) (layer "F.Cu") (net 3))
 (segment (start 126.365 62.23) (end 128.31875 62.23) (width 0.2) (layer "F.Cu") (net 3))
 (segment (start 116.297 74.838) (end 116.297 79.467) (width 0.2) (layer "F.Cu") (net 3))
 (segment (start 128.31875 62.23) (end 128.88875 61.66) (width 0.2) (layer "F.Cu") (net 3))
 (segment (start 102.045 65.85) (end 100.965 64.77) (width 0.2) (layer "F.Cu") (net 3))
 (segment (start 116.297 79.467) (end 118.11 81.28) (width 0.2) (layer "F.Cu") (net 3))
 (segment (start 109.809 65.85) (end 102.045 65.85) (width 0.2) (layer "F.Cu") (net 3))
 (segment (start 125.73 62.865) (end 126.365 62.23) (width 0.2) (layer "F.Cu") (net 3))
 (segment (start 125.73 67.31) (end 125.73 62.865) (width 0.2) (layer "F.Cu") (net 3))
 (segment (start 101.1 70.35) (end 100.965 70.485) (width 0.2) (layer "F.Cu") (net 3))
 (segment (start 109.809 70.35) (end 101.1 70.35) (width 0.2) (layer "F.Cu") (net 3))
 (segment (start 114.935 81.28) (end 110.49 81.28) (width 0.2) (layer "F.Cu") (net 9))
 (segment (start 115.797 57.377) (end 112.395 53.975) (width 0.2) (layer "F.Cu") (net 9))
 (segment (start 115.797 63.362) (end 115.797 57.377) (width 0.2) (layer "F.Cu") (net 9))
 (segment (start 115.797 80.418) (end 114.935 81.28) (width 0.2) (layer "F.Cu") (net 9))
 (segment (start 112.395 53.975) (end 106.72 53.975) (width 0.2) (layer "F.Cu") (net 9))
 (segment (start 115.797 74.838) (end 115.797 80.418) (width 0.2) (layer "F.Cu") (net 9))
 (segment (start 106.72 53.975) (end 106.68 53.935) (width 0.2) (layer "F.Cu") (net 9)))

